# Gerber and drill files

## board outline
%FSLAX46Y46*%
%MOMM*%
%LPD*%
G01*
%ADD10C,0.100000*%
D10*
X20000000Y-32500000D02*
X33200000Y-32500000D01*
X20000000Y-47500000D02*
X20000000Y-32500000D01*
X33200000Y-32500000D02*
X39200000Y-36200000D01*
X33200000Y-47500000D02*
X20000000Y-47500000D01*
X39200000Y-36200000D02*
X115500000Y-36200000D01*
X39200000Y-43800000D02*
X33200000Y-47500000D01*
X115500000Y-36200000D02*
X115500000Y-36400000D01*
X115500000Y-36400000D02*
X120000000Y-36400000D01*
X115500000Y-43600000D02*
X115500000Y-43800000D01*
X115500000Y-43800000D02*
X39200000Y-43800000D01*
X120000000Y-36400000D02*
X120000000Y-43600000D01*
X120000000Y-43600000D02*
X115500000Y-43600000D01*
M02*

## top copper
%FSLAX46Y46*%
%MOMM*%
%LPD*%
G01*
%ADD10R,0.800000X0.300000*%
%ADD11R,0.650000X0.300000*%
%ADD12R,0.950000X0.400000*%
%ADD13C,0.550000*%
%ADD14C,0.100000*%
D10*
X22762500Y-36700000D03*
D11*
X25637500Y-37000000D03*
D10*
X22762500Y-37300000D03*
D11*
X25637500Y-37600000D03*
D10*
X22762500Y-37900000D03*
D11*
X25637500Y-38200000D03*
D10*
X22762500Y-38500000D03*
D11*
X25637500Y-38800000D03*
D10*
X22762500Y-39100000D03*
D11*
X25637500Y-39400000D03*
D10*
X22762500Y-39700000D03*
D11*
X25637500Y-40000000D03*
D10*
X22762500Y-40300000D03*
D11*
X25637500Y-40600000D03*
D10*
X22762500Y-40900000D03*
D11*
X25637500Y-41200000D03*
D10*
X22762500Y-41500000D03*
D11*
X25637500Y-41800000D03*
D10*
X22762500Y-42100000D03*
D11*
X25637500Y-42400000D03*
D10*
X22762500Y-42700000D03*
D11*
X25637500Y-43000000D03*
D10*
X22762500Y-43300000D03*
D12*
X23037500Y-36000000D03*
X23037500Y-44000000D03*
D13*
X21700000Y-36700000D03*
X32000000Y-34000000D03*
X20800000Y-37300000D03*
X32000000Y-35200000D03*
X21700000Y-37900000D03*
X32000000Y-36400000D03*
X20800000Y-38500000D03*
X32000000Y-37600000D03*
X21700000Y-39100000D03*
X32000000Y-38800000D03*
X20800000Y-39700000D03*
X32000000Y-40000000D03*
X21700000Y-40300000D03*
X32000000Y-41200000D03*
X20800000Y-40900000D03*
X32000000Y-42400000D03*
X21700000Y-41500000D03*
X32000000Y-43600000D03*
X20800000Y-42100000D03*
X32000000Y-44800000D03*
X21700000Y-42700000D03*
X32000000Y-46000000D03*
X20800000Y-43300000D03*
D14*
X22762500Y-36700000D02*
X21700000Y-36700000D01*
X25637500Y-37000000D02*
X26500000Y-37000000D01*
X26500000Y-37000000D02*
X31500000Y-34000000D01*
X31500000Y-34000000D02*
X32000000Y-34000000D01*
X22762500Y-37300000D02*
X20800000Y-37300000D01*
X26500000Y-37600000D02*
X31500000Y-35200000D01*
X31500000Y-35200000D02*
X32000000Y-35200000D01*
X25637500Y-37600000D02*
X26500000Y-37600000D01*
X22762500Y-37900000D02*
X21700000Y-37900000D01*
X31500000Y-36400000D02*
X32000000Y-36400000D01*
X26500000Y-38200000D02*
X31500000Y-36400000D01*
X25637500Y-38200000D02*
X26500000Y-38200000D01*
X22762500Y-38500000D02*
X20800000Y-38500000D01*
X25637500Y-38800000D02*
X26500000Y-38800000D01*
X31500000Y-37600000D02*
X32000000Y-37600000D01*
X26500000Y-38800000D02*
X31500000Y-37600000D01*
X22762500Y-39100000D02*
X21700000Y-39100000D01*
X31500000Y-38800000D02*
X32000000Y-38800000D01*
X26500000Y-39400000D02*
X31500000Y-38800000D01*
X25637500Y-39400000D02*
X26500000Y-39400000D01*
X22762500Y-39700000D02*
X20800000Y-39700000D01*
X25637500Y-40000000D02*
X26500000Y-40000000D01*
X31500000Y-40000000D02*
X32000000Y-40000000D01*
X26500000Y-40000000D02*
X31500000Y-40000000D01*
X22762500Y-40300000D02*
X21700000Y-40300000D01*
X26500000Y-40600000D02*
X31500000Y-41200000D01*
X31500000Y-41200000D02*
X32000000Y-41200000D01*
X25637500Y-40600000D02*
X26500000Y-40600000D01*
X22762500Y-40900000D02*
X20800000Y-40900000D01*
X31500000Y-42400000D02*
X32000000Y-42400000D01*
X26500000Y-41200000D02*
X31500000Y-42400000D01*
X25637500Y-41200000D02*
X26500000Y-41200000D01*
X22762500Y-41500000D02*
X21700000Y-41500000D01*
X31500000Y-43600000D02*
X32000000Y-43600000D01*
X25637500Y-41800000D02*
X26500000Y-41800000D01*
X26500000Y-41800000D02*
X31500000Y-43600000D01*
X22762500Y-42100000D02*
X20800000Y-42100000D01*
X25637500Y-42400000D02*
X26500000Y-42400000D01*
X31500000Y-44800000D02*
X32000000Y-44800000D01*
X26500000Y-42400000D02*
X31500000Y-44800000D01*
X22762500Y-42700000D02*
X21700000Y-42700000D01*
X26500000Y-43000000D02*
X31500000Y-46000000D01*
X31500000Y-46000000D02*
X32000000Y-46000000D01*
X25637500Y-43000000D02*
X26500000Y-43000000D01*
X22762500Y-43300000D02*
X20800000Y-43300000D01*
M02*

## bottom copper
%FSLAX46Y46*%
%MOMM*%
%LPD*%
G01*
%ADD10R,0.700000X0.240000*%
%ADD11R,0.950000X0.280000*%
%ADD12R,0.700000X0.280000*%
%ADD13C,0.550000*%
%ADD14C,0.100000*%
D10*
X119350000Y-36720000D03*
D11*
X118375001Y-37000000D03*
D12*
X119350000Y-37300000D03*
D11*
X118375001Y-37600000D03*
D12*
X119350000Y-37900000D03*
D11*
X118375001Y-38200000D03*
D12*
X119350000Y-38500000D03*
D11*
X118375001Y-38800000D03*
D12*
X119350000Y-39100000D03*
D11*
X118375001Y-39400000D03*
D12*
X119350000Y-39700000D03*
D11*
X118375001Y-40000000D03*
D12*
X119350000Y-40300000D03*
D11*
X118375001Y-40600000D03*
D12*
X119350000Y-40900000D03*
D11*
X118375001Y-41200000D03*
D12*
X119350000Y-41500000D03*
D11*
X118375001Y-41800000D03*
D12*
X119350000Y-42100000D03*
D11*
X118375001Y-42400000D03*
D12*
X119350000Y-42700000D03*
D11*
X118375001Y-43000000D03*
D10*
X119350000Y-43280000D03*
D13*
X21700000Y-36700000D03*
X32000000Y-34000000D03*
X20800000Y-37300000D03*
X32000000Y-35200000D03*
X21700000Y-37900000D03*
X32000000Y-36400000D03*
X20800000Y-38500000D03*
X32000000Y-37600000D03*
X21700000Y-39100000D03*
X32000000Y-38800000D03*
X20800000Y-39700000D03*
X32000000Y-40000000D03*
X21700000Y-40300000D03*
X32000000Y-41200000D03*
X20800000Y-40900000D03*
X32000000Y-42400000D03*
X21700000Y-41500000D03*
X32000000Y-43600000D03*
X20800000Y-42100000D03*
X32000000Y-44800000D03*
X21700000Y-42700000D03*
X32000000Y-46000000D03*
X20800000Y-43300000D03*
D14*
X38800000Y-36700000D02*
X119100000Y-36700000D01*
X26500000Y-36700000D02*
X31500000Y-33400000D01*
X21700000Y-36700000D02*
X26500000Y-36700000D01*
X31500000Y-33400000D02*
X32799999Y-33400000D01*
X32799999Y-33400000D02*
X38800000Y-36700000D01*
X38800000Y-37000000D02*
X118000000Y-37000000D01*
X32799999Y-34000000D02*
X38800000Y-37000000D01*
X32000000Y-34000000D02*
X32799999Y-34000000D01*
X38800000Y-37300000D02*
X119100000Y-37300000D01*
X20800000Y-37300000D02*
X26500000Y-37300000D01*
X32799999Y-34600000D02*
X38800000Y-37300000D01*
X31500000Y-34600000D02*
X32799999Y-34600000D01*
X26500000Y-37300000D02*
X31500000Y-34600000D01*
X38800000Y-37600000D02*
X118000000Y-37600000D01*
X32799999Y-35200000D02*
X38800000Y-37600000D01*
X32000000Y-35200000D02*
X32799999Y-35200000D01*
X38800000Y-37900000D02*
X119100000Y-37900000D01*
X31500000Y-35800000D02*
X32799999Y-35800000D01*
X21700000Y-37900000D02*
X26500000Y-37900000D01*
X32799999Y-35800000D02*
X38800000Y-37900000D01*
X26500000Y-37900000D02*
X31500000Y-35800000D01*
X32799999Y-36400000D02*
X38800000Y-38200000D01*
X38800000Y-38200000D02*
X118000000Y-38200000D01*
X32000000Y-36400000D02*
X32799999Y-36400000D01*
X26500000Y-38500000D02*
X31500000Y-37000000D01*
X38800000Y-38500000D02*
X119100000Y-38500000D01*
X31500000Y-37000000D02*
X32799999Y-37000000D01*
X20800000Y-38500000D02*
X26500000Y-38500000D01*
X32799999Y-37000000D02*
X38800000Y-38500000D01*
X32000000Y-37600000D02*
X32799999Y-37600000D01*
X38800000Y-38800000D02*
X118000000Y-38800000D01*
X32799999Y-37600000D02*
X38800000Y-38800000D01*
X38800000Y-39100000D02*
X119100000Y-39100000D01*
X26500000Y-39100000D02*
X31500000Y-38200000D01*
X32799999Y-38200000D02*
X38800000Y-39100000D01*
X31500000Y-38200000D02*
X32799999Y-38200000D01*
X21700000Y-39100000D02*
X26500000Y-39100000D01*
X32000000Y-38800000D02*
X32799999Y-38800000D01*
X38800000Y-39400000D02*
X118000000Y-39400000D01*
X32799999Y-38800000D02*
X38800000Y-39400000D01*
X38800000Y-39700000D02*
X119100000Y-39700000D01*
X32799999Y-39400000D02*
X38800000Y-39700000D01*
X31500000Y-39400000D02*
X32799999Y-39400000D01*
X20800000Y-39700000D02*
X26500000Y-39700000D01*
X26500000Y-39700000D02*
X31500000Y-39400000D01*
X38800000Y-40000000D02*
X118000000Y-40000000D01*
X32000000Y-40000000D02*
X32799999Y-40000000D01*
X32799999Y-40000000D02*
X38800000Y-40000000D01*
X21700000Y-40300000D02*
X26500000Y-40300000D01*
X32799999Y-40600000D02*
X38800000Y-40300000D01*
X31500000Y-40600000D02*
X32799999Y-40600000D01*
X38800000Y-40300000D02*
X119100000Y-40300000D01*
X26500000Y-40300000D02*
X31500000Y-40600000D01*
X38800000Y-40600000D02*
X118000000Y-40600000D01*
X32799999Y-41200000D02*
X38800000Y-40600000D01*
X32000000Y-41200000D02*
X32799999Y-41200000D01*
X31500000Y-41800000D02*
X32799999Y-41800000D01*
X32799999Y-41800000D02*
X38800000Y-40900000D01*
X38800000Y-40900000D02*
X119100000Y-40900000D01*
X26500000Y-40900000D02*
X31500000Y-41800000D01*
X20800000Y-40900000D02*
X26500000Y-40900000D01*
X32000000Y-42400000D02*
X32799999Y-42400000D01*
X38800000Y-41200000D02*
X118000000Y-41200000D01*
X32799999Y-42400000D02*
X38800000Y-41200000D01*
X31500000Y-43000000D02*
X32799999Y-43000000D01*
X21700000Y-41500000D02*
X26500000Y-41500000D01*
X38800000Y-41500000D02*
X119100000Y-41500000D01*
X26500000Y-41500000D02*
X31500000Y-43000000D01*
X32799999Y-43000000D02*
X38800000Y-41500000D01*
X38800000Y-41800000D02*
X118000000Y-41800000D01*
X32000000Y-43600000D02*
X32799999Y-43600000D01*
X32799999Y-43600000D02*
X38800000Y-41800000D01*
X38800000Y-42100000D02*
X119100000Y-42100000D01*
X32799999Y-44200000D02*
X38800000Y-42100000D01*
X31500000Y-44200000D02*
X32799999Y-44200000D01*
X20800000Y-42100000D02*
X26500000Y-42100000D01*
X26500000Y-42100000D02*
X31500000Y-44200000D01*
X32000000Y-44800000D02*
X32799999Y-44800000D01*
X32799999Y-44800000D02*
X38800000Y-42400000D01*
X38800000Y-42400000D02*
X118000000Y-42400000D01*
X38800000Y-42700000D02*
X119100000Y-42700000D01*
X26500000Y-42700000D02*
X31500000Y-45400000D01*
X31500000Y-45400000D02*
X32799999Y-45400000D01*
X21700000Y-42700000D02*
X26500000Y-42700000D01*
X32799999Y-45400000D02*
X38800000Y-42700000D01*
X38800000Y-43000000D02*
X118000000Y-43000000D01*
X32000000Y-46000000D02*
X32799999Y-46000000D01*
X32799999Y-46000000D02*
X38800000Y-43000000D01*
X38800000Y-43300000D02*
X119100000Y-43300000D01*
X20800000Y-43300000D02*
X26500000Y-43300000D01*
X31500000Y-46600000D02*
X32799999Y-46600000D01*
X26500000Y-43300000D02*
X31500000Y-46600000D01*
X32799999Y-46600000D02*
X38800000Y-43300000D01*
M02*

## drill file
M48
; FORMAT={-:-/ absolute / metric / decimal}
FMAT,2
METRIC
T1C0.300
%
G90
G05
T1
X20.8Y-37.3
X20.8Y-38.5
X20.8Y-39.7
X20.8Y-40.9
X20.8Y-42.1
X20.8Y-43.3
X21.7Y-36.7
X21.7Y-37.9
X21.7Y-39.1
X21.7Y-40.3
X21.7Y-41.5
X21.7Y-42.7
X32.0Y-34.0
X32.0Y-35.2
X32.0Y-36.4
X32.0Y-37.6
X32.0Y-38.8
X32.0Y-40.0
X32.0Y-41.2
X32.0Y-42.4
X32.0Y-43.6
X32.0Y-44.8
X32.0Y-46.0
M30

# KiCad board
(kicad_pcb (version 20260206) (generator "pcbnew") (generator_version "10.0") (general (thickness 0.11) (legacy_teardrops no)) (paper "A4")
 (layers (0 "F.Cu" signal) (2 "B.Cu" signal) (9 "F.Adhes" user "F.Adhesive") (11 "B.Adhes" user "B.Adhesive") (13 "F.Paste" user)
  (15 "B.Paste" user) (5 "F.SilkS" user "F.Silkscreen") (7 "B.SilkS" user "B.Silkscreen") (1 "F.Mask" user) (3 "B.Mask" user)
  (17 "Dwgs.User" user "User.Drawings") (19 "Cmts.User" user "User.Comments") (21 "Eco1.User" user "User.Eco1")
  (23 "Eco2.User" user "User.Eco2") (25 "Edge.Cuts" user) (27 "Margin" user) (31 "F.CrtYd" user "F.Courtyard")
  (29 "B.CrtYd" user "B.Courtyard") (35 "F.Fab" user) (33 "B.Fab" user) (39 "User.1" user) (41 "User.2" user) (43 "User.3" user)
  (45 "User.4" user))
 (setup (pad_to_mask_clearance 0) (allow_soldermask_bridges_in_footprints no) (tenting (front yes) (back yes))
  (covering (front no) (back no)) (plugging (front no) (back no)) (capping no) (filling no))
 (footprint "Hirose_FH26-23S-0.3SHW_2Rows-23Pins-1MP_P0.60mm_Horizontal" (layer "F.Cu") (at 24.1625 40)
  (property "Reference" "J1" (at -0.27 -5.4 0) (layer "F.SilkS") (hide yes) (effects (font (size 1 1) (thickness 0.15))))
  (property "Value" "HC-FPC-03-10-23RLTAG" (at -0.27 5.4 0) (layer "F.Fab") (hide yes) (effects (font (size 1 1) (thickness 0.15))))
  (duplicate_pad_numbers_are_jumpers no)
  (pad "1" smd rect (at -1.4 -3.3) (size 0.8 0.3) (layers "F.Cu" "F.Mask" "F.Paste") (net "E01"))
  (pad "2" smd rect (at 1.475 -3) (size 0.65 0.3) (layers "F.Cu" "F.Mask" "F.Paste") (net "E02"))
  (pad "3" smd rect (at -1.4 -2.7) (size 0.8 0.3) (layers "F.Cu" "F.Mask" "F.Paste") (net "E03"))
  (pad "4" smd rect (at 1.475 -2.4) (size 0.65 0.3) (layers "F.Cu" "F.Mask" "F.Paste") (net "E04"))
  (pad "5" smd rect (at -1.4 -2.1) (size 0.8 0.3) (layers "F.Cu" "F.Mask" "F.Paste") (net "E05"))
  (pad "6" smd rect (at 1.475 -1.8) (size 0.65 0.3) (layers "F.Cu" "F.Mask" "F.Paste") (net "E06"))
  (pad "7" smd rect (at -1.4 -1.5) (size 0.8 0.3) (layers "F.Cu" "F.Mask" "F.Paste") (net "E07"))
  (pad "8" smd rect (at 1.475 -1.2) (size 0.65 0.3) (layers "F.Cu" "F.Mask" "F.Paste") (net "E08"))
  (pad "9" smd rect (at -1.4 -0.9) (size 0.8 0.3) (layers "F.Cu" "F.Mask" "F.Paste") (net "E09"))
  (pad "10" smd rect (at 1.475 -0.6) (size 0.65 0.3) (layers "F.Cu" "F.Mask" "F.Paste") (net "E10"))
  (pad "11" smd rect (at -1.4 -0.3) (size 0.8 0.3) (layers "F.Cu" "F.Mask" "F.Paste") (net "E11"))
  (pad "12" smd rect (at 1.475 0) (size 0.65 0.3) (layers "F.Cu" "F.Mask" "F.Paste") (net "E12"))
  (pad "13" smd rect (at -1.4 0.3) (size 0.8 0.3) (layers "F.Cu" "F.Mask" "F.Paste") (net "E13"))
  (pad "14" smd rect (at 1.475 0.6) (size 0.65 0.3) (layers "F.Cu" "F.Mask" "F.Paste") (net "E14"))
  (pad "15" smd rect (at -1.4 0.9) (size 0.8 0.3) (layers "F.Cu" "F.Mask" "F.Paste") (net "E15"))
  (pad "16" smd rect (at 1.475 1.2) (size 0.65 0.3) (layers "F.Cu" "F.Mask" "F.Paste") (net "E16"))
  (pad "17" smd rect (at -1.4 1.5) (size 0.8 0.3) (layers "F.Cu" "F.Mask" "F.Paste") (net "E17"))
  (pad "18" smd rect (at 1.475 1.8) (size 0.65 0.3) (layers "F.Cu" "F.Mask" "F.Paste") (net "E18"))
  (pad "19" smd rect (at -1.4 2.1) (size 0.8 0.3) (layers "F.Cu" "F.Mask" "F.Paste") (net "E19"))
  (pad "20" smd rect (at 1.475 2.4) (size 0.65 0.3) (layers "F.Cu" "F.Mask" "F.Paste") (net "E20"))
  (pad "21" smd rect (at -1.4 2.7) (size 0.8 0.3) (layers "F.Cu" "F.Mask" "F.Paste") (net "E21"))
  (pad "22" smd rect (at 1.475 3) (size 0.65 0.3) (layers "F.Cu" "F.Mask" "F.Paste") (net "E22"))
  (pad "23" smd rect (at -1.4 3.3) (size 0.8 0.3) (layers "F.Cu" "F.Mask" "F.Paste") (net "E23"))
  (pad "MP" smd rect (at -1.125 -4) (size 0.95 0.4) (layers "F.Cu" "F.Mask" "F.Paste"))
  (pad "MP" smd rect (at -1.125 4) (size 0.95 0.4) (layers "F.Cu" "F.Mask" "F.Paste")))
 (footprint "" (layer "B.Cu") (at 118.6 40 180)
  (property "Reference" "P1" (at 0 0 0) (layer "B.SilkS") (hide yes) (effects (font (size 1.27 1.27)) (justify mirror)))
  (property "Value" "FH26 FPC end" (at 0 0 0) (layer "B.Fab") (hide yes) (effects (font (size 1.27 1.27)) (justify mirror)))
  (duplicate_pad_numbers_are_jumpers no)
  (pad "1" smd rect (at -0.75 3.28 180) (size 0.7 0.24) (layers "B.Cu" "B.Mask") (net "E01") (thermal_bridge_angle 45))
  (pad "2" smd rect (at 0.224999 3 180) (size 0.95 0.28) (layers "B.Cu" "B.Mask") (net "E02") (thermal_bridge_angle 45))
  (pad "3" smd rect (at -0.75 2.7 180) (size 0.7 0.28) (layers "B.Cu" "B.Mask") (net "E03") (thermal_bridge_angle 45))
  (pad "4" smd rect (at 0.224999 2.4 180) (size 0.95 0.28) (layers "B.Cu" "B.Mask") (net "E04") (thermal_bridge_angle 45))
  (pad "5" smd rect (at -0.75 2.1 180) (size 0.7 0.28) (layers "B.Cu" "B.Mask") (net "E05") (thermal_bridge_angle 45))
  (pad "6" smd rect (at 0.224999 1.8 180) (size 0.95 0.28) (layers "B.Cu" "B.Mask") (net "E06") (thermal_bridge_angle 45))
  (pad "7" smd rect (at -0.75 1.5 180) (size 0.7 0.28) (layers "B.Cu" "B.Mask") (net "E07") (thermal_bridge_angle 45))
  (pad "8" smd rect (at 0.224999 1.2 180) (size 0.95 0.28) (layers "B.Cu" "B.Mask") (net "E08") (thermal_bridge_angle 45))
  (pad "9" smd rect (at -0.75 0.9 180) (size 0.7 0.28) (layers "B.Cu" "B.Mask") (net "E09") (thermal_bridge_angle 45))
  (pad "10" smd rect (at 0.224999 0.6 180) (size 0.95 0.28) (layers "B.Cu" "B.Mask") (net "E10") (thermal_bridge_angle 45))
  (pad "11" smd rect (at -0.75 0.3 180) (size 0.7 0.28) (layers "B.Cu" "B.Mask") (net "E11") (thermal_bridge_angle 45))
  (pad "12" smd rect (at 0.224999 0 180) (size 0.95 0.28) (layers "B.Cu" "B.Mask") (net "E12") (thermal_bridge_angle 45))
  (pad "13" smd rect (at -0.75 -0.3 180) (size 0.7 0.28) (layers "B.Cu" "B.Mask") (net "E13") (thermal_bridge_angle 45))
  (pad "14" smd rect (at 0.224999 -0.6 180) (size 0.95 0.28) (layers "B.Cu" "B.Mask") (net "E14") (thermal_bridge_angle 45))
  (pad "15" smd rect (at -0.75 -0.9 180) (size 0.7 0.28) (layers "B.Cu" "B.Mask") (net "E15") (thermal_bridge_angle 45))
  (pad "16" smd rect (at 0.224999 -1.2 180) (size 0.95 0.28) (layers "B.Cu" "B.Mask") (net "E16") (thermal_bridge_angle 45))
  (pad "17" smd rect (at -0.75 -1.5 180) (size 0.7 0.28) (layers "B.Cu" "B.Mask") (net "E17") (thermal_bridge_angle 45))
  (pad "18" smd rect (at 0.224999 -1.8 180) (size 0.95 0.28) (layers "B.Cu" "B.Mask") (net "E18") (thermal_bridge_angle 45))
  (pad "19" smd rect (at -0.75 -2.1 180) (size 0.7 0.28) (layers "B.Cu" "B.Mask") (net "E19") (thermal_bridge_angle 45))
  (pad "20" smd rect (at 0.224999 -2.4 180) (size 0.95 0.28) (layers "B.Cu" "B.Mask") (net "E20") (thermal_bridge_angle 45))
  (pad "21" smd rect (at -0.75 -2.7 180) (size 0.7 0.28) (layers "B.Cu" "B.Mask") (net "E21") (thermal_bridge_angle 45))
  (pad "22" smd rect (at 0.224999 -3 180) (size 0.95 0.28) (layers "B.Cu" "B.Mask") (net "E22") (thermal_bridge_angle 45))
  (pad "23" smd rect (at -0.75 -3.28 180) (size 0.7 0.24) (layers "B.Cu" "B.Mask") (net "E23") (thermal_bridge_angle 45)))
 (gr_line (start 20 32.5) (end 33.2 32.5) (stroke (width 0.1) (type default)) (layer "Edge.Cuts"))
 (gr_line (start 20 47.5) (end 20 32.5) (stroke (width 0.1) (type default)) (layer "Edge.Cuts"))
 (gr_line (start 33.2 32.5) (end 39.2 36.2) (stroke (width 0.1) (type default)) (layer "Edge.Cuts"))
 (gr_line (start 33.2 47.5) (end 20 47.5) (stroke (width 0.1) (type default)) (layer "Edge.Cuts"))
 (gr_line (start 39.2 36.2) (end 115.5 36.2) (stroke (width 0.1) (type default)) (layer "Edge.Cuts"))
 (gr_line (start 39.2 43.8) (end 33.2 47.5) (stroke (width 0.1) (type default)) (layer "Edge.Cuts"))
 (gr_line (start 115.5 36.2) (end 115.5 36.4) (stroke (width 0.1) (type default)) (layer "Edge.Cuts"))
 (gr_line (start 115.5 36.4) (end 120 36.4) (stroke (width 0.1) (type default)) (layer "Edge.Cuts"))
 (gr_line (start 115.5 43.6) (end 115.5 43.8) (stroke (width 0.1) (type default)) (layer "Edge.Cuts"))
 (gr_line (start 115.5 43.8) (end 39.2 43.8) (stroke (width 0.1) (type default)) (layer "Edge.Cuts"))
 (gr_line (start 120 36.4) (end 120 43.6) (stroke (width 0.1) (type default)) (layer "Edge.Cuts"))
 (gr_line (start 120 43.6) (end 115.5 43.6) (stroke (width 0.1) (type default)) (layer "Edge.Cuts"))
 (segment (start 22.7625 36.7) (end 21.7 36.7) (width 0.1) (layer "F.Cu") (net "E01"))
 (via (at 21.7 36.7) (size 0.55) (drill 0.3) (layers "F.Cu" "B.Cu") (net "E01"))
 (segment (start 38.8 36.7) (end 119.1 36.7) (width 0.1) (layer "B.Cu") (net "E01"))
 (segment (start 26.5 36.7) (end 31.5 33.4) (width 0.1) (layer "B.Cu") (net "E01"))
 (segment (start 21.7 36.7) (end 26.5 36.7) (width 0.1) (layer "B.Cu") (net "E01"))
 (segment (start 31.5 33.4) (end 32.799999 33.4) (width 0.1) (layer "B.Cu") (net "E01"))
 (segment (start 32.799999 33.4) (end 38.8 36.7) (width 0.1) (layer "B.Cu") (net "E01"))
 (segment (start 25.6375 37) (end 26.5 37) (width 0.1) (layer "F.Cu") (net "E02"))
 (segment (start 26.5 37) (end 31.5 34) (width 0.1) (layer "F.Cu") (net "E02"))
 (segment (start 31.5 34) (end 32 34) (width 0.1) (layer "F.Cu") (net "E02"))
 (via (at 32 34) (size 0.55) (drill 0.3) (layers "F.Cu" "B.Cu") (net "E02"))
 (segment (start 38.8 37) (end 118 37) (width 0.1) (layer "B.Cu") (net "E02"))
 (segment (start 32.799999 34) (end 38.8 37) (width 0.1) (layer "B.Cu") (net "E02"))
 (segment (start 32 34) (end 32.799999 34) (width 0.1) (layer "B.Cu") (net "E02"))
 (segment (start 22.7625 37.3) (end 20.8 37.3) (width 0.1) (layer "F.Cu") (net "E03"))
 (via (at 20.8 37.3) (size 0.55) (drill 0.3) (layers "F.Cu" "B.Cu") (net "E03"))
 (segment (start 38.8 37.3) (end 119.1 37.3) (width 0.1) (layer "B.Cu") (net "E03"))
 (segment (start 20.8 37.3) (end 26.5 37.3) (width 0.1) (layer "B.Cu") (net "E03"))
 (segment (start 32.799999 34.6) (end 38.8 37.3) (width 0.1) (layer "B.Cu") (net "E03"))
 (segment (start 31.5 34.6) (end 32.799999 34.6) (width 0.1) (layer "B.Cu") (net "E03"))
 (segment (start 26.5 37.3) (end 31.5 34.6) (width 0.1) (layer "B.Cu") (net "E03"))
 (segment (start 26.5 37.6) (end 31.5 35.2) (width 0.1) (layer "F.Cu") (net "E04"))
 (segment (start 31.5 35.2) (end 32 35.2) (width 0.1) (layer "F.Cu") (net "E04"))
 (segment (start 25.6375 37.6) (end 26.5 37.6) (width 0.1) (layer "F.Cu") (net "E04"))
 (via (at 32 35.2) (size 0.55) (drill 0.3) (layers "F.Cu" "B.Cu") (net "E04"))
 (segment (start 38.8 37.6) (end 118 37.6) (width 0.1) (layer "B.Cu") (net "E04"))
 (segment (start 32.799999 35.2) (end 38.8 37.6) (width 0.1) (layer "B.Cu") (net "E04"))
 (segment (start 32 35.2) (end 32.799999 35.2) (width 0.1) (layer "B.Cu") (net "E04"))
 (segment (start 22.7625 37.9) (end 21.7 37.9) (width 0.1) (layer "F.Cu") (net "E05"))
 (via (at 21.7 37.9) (size 0.55) (drill 0.3) (layers "F.Cu" "B.Cu") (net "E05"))
 (segment (start 38.8 37.9) (end 119.1 37.9) (width 0.1) (layer "B.Cu") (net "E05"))
 (segment (start 31.5 35.8) (end 32.799999 35.8) (width 0.1) (layer "B.Cu") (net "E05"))
 (segment (start 21.7 37.9) (end 26.5 37.9) (width 0.1) (layer "B.Cu") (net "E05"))
 (segment (start 32.799999 35.8) (end 38.8 37.9) (width 0.1) (layer "B.Cu") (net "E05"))
 (segment (start 26.5 37.9) (end 31.5 35.8) (width 0.1) (layer "B.Cu") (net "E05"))
 (segment (start 31.5 36.4) (end 32 36.4) (width 0.1) (layer "F.Cu") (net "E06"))
 (segment (start 26.5 38.2) (end 31.5 36.4) (width 0.1) (layer "F.Cu") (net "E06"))
 (segment (start 25.6375 38.2) (end 26.5 38.2) (width 0.1) (layer "F.Cu") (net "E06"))
 (via (at 32 36.4) (size 0.55) (drill 0.3) (layers "F.Cu" "B.Cu") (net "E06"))
 (segment (start 32.799999 36.4) (end 38.8 38.2) (width 0.1) (layer "B.Cu") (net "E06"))
 (segment (start 38.8 38.2) (end 118 38.2) (width 0.1) (layer "B.Cu") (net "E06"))
 (segment (start 32 36.4) (end 32.799999 36.4) (width 0.1) (layer "B.Cu") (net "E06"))
 (segment (start 22.7625 38.5) (end 20.8 38.5) (width 0.1) (layer "F.Cu") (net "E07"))
 (via (at 20.8 38.5) (size 0.55) (drill 0.3) (layers "F.Cu" "B.Cu") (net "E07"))
 (segment (start 26.5 38.5) (end 31.5 37) (width 0.1) (layer "B.Cu") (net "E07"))
 (segment (start 38.8 38.5) (end 119.1 38.5) (width 0.1) (layer "B.Cu") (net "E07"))
 (segment (start 31.5 37) (end 32.799999 37) (width 0.1) (layer "B.Cu") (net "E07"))
 (segment (start 20.8 38.5) (end 26.5 38.5) (width 0.1) (layer "B.Cu") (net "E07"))
 (segment (start 32.799999 37) (end 38.8 38.5) (width 0.1) (layer "B.Cu") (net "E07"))
 (segment (start 25.6375 38.8) (end 26.5 38.8) (width 0.1) (layer "F.Cu") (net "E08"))
 (segment (start 31.5 37.6) (end 32 37.6) (width 0.1) (layer "F.Cu") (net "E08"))
 (segment (start 26.5 38.8) (end 31.5 37.6) (width 0.1) (layer "F.Cu") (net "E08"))
 (via (at 32 37.6) (size 0.55) (drill 0.3) (layers "F.Cu" "B.Cu") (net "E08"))
 (segment (start 32 37.6) (end 32.799999 37.6) (width 0.1) (layer "B.Cu") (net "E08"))
 (segment (start 38.8 38.8) (end 118 38.8) (width 0.1) (layer "B.Cu") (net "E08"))
 (segment (start 32.799999 37.6) (end 38.8 38.8) (width 0.1) (layer "B.Cu") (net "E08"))
 (segment (start 22.7625 39.1) (end 21.7 39.1) (width 0.1) (layer "F.Cu") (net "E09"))
 (via (at 21.7 39.1) (size 0.55) (drill 0.3) (layers "F.Cu" "B.Cu") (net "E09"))
 (segment (start 38.8 39.1) (end 119.1 39.1) (width 0.1) (layer "B.Cu") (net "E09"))
 (segment (start 26.5 39.1) (end 31.5 38.2) (width 0.1) (layer "B.Cu") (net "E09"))
 (segment (start 32.799999 38.2) (end 38.8 39.1) (width 0.1) (layer "B.Cu") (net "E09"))
 (segment (start 31.5 38.2) (end 32.799999 38.2) (width 0.1) (layer "B.Cu") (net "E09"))
 (segment (start 21.7 39.1) (end 26.5 39.1) (width 0.1) (layer "B.Cu") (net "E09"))
 (segment (start 31.5 38.8) (end 32 38.8) (width 0.1) (layer "F.Cu") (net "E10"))
 (segment (start 26.5 39.4) (end 31.5 38.8) (width 0.1) (layer "F.Cu") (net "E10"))
 (segment (start 25.6375 39.4) (end 26.5 39.4) (width 0.1) (layer "F.Cu") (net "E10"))
 (via (at 32 38.8) (size 0.55) (drill 0.3) (layers "F.Cu" "B.Cu") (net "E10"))
 (segment (start 32 38.8) (end 32.799999 38.8) (width 0.1) (layer "B.Cu") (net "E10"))
 (segment (start 38.8 39.4) (end 118 39.4) (width 0.1) (layer "B.Cu") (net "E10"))
 (segment (start 32.799999 38.8) (end 38.8 39.4) (width 0.1) (layer "B.Cu") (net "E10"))
 (segment (start 22.7625 39.7) (end 20.8 39.7) (width 0.1) (layer "F.Cu") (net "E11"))
 (via (at 20.8 39.7) (size 0.55) (drill 0.3) (layers "F.Cu" "B.Cu") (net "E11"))
 (segment (start 38.8 39.7) (end 119.1 39.7) (width 0.1) (layer "B.Cu") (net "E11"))
 (segment (start 32.799999 39.4) (end 38.8 39.7) (width 0.1) (layer "B.Cu") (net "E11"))
 (segment (start 31.5 39.4) (end 32.799999 39.4) (width 0.1) (layer "B.Cu") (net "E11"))
 (segment (start 20.8 39.7) (end 26.5 39.7) (width 0.1) (layer "B.Cu") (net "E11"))
 (segment (start 26.5 39.7) (end 31.5 39.4) (width 0.1) (layer "B.Cu") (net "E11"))
 (segment (start 25.6375 40) (end 26.5 40) (width 0.1) (layer "F.Cu") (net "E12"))
 (segment (start 31.5 40) (end 32 40) (width 0.1) (layer "F.Cu") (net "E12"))
 (segment (start 26.5 40) (end 31.5 40) (width 0.1) (layer "F.Cu") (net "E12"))
 (via (at 32 40) (size 0.55) (drill 0.3) (layers "F.Cu" "B.Cu") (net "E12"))
 (segment (start 38.8 40) (end 118 40) (width 0.1) (layer "B.Cu") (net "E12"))
 (segment (start 32 40) (end 32.799999 40) (width 0.1) (layer "B.Cu") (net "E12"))
 (segment (start 32.799999 40) (end 38.8 40) (width 0.1) (layer "B.Cu") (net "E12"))
 (segment (start 22.7625 40.3) (end 21.7 40.3) (width 0.1) (layer "F.Cu") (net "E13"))
 (via (at 21.7 40.3) (size 0.55) (drill 0.3) (layers "F.Cu" "B.Cu") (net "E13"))
 (segment (start 21.7 40.3) (end 26.5 40.3) (width 0.1) (layer "B.Cu") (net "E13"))
 (segment (start 32.799999 40.6) (end 38.8 40.3) (width 0.1) (layer "B.Cu") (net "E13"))
 (segment (start 31.5 40.6) (end 32.799999 40.6) (width 0.1) (layer "B.Cu") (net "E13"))
 (segment (start 38.8 40.3) (end 119.1 40.3) (width 0.1) (layer "B.Cu") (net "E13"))
 (segment (start 26.5 40.3) (end 31.5 40.6) (width 0.1) (layer "B.Cu") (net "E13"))
 (segment (start 26.5 40.6) (end 31.5 41.2) (width 0.1) (layer "F.Cu") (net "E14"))
 (segment (start 31.5 41.2) (end 32 41.2) (width 0.1) (layer "F.Cu") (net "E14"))
 (segment (start 25.6375 40.6) (end 26.5 40.6) (width 0.1) (layer "F.Cu") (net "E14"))
 (via (at 32 41.2) (size 0.55) (drill 0.3) (layers "F.Cu" "B.Cu") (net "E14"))
 (segment (start 38.8 40.6) (end 118 40.6) (width 0.1) (layer "B.Cu") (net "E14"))
 (segment (start 32.799999 41.2) (end 38.8 40.6) (width 0.1) (layer "B.Cu") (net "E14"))
 (segment (start 32 41.2) (end 32.799999 41.2) (width 0.1) (layer "B.Cu") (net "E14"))
 (segment (start 22.7625 40.9) (end 20.8 40.9) (width 0.1) (layer "F.Cu") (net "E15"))
 (via (at 20.8 40.9) (size 0.55) (drill 0.3) (layers "F.Cu" "B.Cu") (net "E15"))
 (segment (start 31.5 41.8) (end 32.799999 41.8) (width 0.1) (layer "B.Cu") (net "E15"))
 (segment (start 32.799999 41.8) (end 38.8 40.9) (width 0.1) (layer "B.Cu") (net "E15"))
 (segment (start 38.8 40.9) (end 119.1 40.9) (width 0.1) (layer "B.Cu") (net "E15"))
 (segment (start 26.5 40.9) (end 31.5 41.8) (width 0.1) (layer "B.Cu") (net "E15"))
 (segment (start 20.8 40.9) (end 26.5 40.9) (width 0.1) (layer "B.Cu") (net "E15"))
 (segment (start 31.5 42.4) (end 32 42.4) (width 0.1) (layer "F.Cu") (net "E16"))
 (segment (start 26.5 41.2) (end 31.5 42.4) (width 0.1) (layer "F.Cu") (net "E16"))
 (segment (start 25.6375 41.2) (end 26.5 41.2) (width 0.1) (layer "F.Cu") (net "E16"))
 (via (at 32 42.4) (size 0.55) (drill 0.3) (layers "F.Cu" "B.Cu") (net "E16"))
 (segment (start 32 42.4) (end 32.799999 42.4) (width 0.1) (layer "B.Cu") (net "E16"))
 (segment (start 38.8 41.2) (end 118 41.2) (width 0.1) (layer "B.Cu") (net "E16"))
 (segment (start 32.799999 42.4) (end 38.8 41.2) (width 0.1) (layer "B.Cu") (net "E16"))
 (segment (start 22.7625 41.5) (end 21.7 41.5) (width 0.1) (layer "F.Cu") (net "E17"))
 (via (at 21.7 41.5) (size 0.55) (drill 0.3) (layers "F.Cu" "B.Cu") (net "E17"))
 (segment (start 31.5 43) (end 32.799999 43) (width 0.1) (layer "B.Cu") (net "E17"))
 (segment (start 21.7 41.5) (end 26.5 41.5) (width 0.1) (layer "B.Cu") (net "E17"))
 (segment (start 38.8 41.5) (end 119.1 41.5) (width 0.1) (layer "B.Cu") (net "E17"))
 (segment (start 26.5 41.5) (end 31.5 43) (width 0.1) (layer "B.Cu") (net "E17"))
 (segment (start 32.799999 43) (end 38.8 41.5) (width 0.1) (layer "B.Cu") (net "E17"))
 (segment (start 31.5 43.6) (end 32 43.6) (width 0.1) (layer "F.Cu") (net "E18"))
 (segment (start 25.6375 41.8) (end 26.5 41.8) (width 0.1) (layer "F.Cu") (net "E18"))
 (segment (start 26.5 41.8) (end 31.5 43.6) (width 0.1) (layer "F.Cu") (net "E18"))
 (via (at 32 43.6) (size 0.55) (drill 0.3) (layers "F.Cu" "B.Cu") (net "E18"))
 (segment (start 38.8 41.8) (end 118 41.8) (width 0.1) (layer "B.Cu") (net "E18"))
 (segment (start 32 43.6) (end 32.799999 43.6) (width 0.1) (layer "B.Cu") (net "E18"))
 (segment (start 32.799999 43.6) (end 38.8 41.8) (width 0.1) (layer "B.Cu") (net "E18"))
 (segment (start 22.7625 42.1) (end 20.8 42.1) (width 0.1) (layer "F.Cu") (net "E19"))
 (via (at 20.8 42.1) (size 0.55) (drill 0.3) (layers "F.Cu" "B.Cu") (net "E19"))
 (segment (start 38.8 42.1) (end 119.1 42.1) (width 0.1) (layer "B.Cu") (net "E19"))
 (segment (start 32.799999 44.2) (end 38.8 42.1) (width 0.1) (layer "B.Cu") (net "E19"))
 (segment (start 31.5 44.2) (end 32.799999 44.2) (width 0.1) (layer "B.Cu") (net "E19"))
 (segment (start 20.8 42.1) (end 26.5 42.1) (width 0.1) (layer "B.Cu") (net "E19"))
 (segment (start 26.5 42.1) (end 31.5 44.2) (width 0.1) (layer "B.Cu") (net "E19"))
 (segment (start 25.6375 42.4) (end 26.5 42.4) (width 0.1) (layer "F.Cu") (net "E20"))
 (segment (start 31.5 44.8) (end 32 44.8) (width 0.1) (layer "F.Cu") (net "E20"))
 (segment (start 26.5 42.4) (end 31.5 44.8) (width 0.1) (layer "F.Cu") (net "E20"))
 (via (at 32 44.8) (size 0.55) (drill 0.3) (layers "F.Cu" "B.Cu") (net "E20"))
 (segment (start 32 44.8) (end 32.799999 44.8) (width 0.1) (layer "B.Cu") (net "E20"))
 (segment (start 32.799999 44.8) (end 38.8 42.4) (width 0.1) (layer "B.Cu") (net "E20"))
 (segment (start 38.8 42.4) (end 118 42.4) (width 0.1) (layer "B.Cu") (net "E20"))
 (segment (start 22.7625 42.7) (end 21.7 42.7) (width 0.1) (layer "F.Cu") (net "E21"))
 (via (at 21.7 42.7) (size 0.55) (drill 0.3) (layers "F.Cu" "B.Cu") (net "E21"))
 (segment (start 38.8 42.7) (end 119.1 42.7) (width 0.1) (layer "B.Cu") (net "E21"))
 (segment (start 26.5 42.7) (end 31.5 45.4) (width 0.1) (layer "B.Cu") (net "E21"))
 (segment (start 31.5 45.4) (end 32.799999 45.4) (width 0.1) (layer "B.Cu") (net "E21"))
 (segment (start 21.7 42.7) (end 26.5 42.7) (width 0.1) (layer "B.Cu") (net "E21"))
 (segment (start 32.799999 45.4) (end 38.8 42.7) (width 0.1) (layer "B.Cu") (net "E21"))
 (segment (start 26.5 43) (end 31.5 46) (width 0.1) (layer "F.Cu") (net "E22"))
 (segment (start 31.5 46) (end 32 46) (width 0.1) (layer "F.Cu") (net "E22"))
 (segment (start 25.6375 43) (end 26.5 43) (width 0.1) (layer "F.Cu") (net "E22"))
 (via (at 32 46) (size 0.55) (drill 0.3) (layers "F.Cu" "B.Cu") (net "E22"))
 (segment (start 38.8 43) (end 118 43) (width 0.1) (layer "B.Cu") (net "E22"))
 (segment (start 32 46) (end 32.799999 46) (width 0.1) (layer "B.Cu") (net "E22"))
 (segment (start 32.799999 46) (end 38.8 43) (width 0.1) (layer "B.Cu") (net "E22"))
 (segment (start 22.7625 43.3) (end 20.8 43.3) (width 0.1) (layer "F.Cu") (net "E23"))
 (via (at 20.8 43.3) (size 0.55) (drill 0.3) (layers "F.Cu" "B.Cu") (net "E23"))
 (segment (start 38.8 43.3) (end 119.1 43.3) (width 0.1) (layer "B.Cu") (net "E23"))
 (segment (start 20.8 43.3) (end 26.5 43.3) (width 0.1) (layer "B.Cu") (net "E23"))
 (segment (start 31.5 46.6) (end 32.799999 46.6) (width 0.1) (layer "B.Cu") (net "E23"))
 (segment (start 26.5 43.3) (end 31.5 46.6) (width 0.1) (layer "B.Cu") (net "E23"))
 (segment (start 32.799999 46.6) (end 38.8 43.3) (width 0.1) (layer "B.Cu") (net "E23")))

